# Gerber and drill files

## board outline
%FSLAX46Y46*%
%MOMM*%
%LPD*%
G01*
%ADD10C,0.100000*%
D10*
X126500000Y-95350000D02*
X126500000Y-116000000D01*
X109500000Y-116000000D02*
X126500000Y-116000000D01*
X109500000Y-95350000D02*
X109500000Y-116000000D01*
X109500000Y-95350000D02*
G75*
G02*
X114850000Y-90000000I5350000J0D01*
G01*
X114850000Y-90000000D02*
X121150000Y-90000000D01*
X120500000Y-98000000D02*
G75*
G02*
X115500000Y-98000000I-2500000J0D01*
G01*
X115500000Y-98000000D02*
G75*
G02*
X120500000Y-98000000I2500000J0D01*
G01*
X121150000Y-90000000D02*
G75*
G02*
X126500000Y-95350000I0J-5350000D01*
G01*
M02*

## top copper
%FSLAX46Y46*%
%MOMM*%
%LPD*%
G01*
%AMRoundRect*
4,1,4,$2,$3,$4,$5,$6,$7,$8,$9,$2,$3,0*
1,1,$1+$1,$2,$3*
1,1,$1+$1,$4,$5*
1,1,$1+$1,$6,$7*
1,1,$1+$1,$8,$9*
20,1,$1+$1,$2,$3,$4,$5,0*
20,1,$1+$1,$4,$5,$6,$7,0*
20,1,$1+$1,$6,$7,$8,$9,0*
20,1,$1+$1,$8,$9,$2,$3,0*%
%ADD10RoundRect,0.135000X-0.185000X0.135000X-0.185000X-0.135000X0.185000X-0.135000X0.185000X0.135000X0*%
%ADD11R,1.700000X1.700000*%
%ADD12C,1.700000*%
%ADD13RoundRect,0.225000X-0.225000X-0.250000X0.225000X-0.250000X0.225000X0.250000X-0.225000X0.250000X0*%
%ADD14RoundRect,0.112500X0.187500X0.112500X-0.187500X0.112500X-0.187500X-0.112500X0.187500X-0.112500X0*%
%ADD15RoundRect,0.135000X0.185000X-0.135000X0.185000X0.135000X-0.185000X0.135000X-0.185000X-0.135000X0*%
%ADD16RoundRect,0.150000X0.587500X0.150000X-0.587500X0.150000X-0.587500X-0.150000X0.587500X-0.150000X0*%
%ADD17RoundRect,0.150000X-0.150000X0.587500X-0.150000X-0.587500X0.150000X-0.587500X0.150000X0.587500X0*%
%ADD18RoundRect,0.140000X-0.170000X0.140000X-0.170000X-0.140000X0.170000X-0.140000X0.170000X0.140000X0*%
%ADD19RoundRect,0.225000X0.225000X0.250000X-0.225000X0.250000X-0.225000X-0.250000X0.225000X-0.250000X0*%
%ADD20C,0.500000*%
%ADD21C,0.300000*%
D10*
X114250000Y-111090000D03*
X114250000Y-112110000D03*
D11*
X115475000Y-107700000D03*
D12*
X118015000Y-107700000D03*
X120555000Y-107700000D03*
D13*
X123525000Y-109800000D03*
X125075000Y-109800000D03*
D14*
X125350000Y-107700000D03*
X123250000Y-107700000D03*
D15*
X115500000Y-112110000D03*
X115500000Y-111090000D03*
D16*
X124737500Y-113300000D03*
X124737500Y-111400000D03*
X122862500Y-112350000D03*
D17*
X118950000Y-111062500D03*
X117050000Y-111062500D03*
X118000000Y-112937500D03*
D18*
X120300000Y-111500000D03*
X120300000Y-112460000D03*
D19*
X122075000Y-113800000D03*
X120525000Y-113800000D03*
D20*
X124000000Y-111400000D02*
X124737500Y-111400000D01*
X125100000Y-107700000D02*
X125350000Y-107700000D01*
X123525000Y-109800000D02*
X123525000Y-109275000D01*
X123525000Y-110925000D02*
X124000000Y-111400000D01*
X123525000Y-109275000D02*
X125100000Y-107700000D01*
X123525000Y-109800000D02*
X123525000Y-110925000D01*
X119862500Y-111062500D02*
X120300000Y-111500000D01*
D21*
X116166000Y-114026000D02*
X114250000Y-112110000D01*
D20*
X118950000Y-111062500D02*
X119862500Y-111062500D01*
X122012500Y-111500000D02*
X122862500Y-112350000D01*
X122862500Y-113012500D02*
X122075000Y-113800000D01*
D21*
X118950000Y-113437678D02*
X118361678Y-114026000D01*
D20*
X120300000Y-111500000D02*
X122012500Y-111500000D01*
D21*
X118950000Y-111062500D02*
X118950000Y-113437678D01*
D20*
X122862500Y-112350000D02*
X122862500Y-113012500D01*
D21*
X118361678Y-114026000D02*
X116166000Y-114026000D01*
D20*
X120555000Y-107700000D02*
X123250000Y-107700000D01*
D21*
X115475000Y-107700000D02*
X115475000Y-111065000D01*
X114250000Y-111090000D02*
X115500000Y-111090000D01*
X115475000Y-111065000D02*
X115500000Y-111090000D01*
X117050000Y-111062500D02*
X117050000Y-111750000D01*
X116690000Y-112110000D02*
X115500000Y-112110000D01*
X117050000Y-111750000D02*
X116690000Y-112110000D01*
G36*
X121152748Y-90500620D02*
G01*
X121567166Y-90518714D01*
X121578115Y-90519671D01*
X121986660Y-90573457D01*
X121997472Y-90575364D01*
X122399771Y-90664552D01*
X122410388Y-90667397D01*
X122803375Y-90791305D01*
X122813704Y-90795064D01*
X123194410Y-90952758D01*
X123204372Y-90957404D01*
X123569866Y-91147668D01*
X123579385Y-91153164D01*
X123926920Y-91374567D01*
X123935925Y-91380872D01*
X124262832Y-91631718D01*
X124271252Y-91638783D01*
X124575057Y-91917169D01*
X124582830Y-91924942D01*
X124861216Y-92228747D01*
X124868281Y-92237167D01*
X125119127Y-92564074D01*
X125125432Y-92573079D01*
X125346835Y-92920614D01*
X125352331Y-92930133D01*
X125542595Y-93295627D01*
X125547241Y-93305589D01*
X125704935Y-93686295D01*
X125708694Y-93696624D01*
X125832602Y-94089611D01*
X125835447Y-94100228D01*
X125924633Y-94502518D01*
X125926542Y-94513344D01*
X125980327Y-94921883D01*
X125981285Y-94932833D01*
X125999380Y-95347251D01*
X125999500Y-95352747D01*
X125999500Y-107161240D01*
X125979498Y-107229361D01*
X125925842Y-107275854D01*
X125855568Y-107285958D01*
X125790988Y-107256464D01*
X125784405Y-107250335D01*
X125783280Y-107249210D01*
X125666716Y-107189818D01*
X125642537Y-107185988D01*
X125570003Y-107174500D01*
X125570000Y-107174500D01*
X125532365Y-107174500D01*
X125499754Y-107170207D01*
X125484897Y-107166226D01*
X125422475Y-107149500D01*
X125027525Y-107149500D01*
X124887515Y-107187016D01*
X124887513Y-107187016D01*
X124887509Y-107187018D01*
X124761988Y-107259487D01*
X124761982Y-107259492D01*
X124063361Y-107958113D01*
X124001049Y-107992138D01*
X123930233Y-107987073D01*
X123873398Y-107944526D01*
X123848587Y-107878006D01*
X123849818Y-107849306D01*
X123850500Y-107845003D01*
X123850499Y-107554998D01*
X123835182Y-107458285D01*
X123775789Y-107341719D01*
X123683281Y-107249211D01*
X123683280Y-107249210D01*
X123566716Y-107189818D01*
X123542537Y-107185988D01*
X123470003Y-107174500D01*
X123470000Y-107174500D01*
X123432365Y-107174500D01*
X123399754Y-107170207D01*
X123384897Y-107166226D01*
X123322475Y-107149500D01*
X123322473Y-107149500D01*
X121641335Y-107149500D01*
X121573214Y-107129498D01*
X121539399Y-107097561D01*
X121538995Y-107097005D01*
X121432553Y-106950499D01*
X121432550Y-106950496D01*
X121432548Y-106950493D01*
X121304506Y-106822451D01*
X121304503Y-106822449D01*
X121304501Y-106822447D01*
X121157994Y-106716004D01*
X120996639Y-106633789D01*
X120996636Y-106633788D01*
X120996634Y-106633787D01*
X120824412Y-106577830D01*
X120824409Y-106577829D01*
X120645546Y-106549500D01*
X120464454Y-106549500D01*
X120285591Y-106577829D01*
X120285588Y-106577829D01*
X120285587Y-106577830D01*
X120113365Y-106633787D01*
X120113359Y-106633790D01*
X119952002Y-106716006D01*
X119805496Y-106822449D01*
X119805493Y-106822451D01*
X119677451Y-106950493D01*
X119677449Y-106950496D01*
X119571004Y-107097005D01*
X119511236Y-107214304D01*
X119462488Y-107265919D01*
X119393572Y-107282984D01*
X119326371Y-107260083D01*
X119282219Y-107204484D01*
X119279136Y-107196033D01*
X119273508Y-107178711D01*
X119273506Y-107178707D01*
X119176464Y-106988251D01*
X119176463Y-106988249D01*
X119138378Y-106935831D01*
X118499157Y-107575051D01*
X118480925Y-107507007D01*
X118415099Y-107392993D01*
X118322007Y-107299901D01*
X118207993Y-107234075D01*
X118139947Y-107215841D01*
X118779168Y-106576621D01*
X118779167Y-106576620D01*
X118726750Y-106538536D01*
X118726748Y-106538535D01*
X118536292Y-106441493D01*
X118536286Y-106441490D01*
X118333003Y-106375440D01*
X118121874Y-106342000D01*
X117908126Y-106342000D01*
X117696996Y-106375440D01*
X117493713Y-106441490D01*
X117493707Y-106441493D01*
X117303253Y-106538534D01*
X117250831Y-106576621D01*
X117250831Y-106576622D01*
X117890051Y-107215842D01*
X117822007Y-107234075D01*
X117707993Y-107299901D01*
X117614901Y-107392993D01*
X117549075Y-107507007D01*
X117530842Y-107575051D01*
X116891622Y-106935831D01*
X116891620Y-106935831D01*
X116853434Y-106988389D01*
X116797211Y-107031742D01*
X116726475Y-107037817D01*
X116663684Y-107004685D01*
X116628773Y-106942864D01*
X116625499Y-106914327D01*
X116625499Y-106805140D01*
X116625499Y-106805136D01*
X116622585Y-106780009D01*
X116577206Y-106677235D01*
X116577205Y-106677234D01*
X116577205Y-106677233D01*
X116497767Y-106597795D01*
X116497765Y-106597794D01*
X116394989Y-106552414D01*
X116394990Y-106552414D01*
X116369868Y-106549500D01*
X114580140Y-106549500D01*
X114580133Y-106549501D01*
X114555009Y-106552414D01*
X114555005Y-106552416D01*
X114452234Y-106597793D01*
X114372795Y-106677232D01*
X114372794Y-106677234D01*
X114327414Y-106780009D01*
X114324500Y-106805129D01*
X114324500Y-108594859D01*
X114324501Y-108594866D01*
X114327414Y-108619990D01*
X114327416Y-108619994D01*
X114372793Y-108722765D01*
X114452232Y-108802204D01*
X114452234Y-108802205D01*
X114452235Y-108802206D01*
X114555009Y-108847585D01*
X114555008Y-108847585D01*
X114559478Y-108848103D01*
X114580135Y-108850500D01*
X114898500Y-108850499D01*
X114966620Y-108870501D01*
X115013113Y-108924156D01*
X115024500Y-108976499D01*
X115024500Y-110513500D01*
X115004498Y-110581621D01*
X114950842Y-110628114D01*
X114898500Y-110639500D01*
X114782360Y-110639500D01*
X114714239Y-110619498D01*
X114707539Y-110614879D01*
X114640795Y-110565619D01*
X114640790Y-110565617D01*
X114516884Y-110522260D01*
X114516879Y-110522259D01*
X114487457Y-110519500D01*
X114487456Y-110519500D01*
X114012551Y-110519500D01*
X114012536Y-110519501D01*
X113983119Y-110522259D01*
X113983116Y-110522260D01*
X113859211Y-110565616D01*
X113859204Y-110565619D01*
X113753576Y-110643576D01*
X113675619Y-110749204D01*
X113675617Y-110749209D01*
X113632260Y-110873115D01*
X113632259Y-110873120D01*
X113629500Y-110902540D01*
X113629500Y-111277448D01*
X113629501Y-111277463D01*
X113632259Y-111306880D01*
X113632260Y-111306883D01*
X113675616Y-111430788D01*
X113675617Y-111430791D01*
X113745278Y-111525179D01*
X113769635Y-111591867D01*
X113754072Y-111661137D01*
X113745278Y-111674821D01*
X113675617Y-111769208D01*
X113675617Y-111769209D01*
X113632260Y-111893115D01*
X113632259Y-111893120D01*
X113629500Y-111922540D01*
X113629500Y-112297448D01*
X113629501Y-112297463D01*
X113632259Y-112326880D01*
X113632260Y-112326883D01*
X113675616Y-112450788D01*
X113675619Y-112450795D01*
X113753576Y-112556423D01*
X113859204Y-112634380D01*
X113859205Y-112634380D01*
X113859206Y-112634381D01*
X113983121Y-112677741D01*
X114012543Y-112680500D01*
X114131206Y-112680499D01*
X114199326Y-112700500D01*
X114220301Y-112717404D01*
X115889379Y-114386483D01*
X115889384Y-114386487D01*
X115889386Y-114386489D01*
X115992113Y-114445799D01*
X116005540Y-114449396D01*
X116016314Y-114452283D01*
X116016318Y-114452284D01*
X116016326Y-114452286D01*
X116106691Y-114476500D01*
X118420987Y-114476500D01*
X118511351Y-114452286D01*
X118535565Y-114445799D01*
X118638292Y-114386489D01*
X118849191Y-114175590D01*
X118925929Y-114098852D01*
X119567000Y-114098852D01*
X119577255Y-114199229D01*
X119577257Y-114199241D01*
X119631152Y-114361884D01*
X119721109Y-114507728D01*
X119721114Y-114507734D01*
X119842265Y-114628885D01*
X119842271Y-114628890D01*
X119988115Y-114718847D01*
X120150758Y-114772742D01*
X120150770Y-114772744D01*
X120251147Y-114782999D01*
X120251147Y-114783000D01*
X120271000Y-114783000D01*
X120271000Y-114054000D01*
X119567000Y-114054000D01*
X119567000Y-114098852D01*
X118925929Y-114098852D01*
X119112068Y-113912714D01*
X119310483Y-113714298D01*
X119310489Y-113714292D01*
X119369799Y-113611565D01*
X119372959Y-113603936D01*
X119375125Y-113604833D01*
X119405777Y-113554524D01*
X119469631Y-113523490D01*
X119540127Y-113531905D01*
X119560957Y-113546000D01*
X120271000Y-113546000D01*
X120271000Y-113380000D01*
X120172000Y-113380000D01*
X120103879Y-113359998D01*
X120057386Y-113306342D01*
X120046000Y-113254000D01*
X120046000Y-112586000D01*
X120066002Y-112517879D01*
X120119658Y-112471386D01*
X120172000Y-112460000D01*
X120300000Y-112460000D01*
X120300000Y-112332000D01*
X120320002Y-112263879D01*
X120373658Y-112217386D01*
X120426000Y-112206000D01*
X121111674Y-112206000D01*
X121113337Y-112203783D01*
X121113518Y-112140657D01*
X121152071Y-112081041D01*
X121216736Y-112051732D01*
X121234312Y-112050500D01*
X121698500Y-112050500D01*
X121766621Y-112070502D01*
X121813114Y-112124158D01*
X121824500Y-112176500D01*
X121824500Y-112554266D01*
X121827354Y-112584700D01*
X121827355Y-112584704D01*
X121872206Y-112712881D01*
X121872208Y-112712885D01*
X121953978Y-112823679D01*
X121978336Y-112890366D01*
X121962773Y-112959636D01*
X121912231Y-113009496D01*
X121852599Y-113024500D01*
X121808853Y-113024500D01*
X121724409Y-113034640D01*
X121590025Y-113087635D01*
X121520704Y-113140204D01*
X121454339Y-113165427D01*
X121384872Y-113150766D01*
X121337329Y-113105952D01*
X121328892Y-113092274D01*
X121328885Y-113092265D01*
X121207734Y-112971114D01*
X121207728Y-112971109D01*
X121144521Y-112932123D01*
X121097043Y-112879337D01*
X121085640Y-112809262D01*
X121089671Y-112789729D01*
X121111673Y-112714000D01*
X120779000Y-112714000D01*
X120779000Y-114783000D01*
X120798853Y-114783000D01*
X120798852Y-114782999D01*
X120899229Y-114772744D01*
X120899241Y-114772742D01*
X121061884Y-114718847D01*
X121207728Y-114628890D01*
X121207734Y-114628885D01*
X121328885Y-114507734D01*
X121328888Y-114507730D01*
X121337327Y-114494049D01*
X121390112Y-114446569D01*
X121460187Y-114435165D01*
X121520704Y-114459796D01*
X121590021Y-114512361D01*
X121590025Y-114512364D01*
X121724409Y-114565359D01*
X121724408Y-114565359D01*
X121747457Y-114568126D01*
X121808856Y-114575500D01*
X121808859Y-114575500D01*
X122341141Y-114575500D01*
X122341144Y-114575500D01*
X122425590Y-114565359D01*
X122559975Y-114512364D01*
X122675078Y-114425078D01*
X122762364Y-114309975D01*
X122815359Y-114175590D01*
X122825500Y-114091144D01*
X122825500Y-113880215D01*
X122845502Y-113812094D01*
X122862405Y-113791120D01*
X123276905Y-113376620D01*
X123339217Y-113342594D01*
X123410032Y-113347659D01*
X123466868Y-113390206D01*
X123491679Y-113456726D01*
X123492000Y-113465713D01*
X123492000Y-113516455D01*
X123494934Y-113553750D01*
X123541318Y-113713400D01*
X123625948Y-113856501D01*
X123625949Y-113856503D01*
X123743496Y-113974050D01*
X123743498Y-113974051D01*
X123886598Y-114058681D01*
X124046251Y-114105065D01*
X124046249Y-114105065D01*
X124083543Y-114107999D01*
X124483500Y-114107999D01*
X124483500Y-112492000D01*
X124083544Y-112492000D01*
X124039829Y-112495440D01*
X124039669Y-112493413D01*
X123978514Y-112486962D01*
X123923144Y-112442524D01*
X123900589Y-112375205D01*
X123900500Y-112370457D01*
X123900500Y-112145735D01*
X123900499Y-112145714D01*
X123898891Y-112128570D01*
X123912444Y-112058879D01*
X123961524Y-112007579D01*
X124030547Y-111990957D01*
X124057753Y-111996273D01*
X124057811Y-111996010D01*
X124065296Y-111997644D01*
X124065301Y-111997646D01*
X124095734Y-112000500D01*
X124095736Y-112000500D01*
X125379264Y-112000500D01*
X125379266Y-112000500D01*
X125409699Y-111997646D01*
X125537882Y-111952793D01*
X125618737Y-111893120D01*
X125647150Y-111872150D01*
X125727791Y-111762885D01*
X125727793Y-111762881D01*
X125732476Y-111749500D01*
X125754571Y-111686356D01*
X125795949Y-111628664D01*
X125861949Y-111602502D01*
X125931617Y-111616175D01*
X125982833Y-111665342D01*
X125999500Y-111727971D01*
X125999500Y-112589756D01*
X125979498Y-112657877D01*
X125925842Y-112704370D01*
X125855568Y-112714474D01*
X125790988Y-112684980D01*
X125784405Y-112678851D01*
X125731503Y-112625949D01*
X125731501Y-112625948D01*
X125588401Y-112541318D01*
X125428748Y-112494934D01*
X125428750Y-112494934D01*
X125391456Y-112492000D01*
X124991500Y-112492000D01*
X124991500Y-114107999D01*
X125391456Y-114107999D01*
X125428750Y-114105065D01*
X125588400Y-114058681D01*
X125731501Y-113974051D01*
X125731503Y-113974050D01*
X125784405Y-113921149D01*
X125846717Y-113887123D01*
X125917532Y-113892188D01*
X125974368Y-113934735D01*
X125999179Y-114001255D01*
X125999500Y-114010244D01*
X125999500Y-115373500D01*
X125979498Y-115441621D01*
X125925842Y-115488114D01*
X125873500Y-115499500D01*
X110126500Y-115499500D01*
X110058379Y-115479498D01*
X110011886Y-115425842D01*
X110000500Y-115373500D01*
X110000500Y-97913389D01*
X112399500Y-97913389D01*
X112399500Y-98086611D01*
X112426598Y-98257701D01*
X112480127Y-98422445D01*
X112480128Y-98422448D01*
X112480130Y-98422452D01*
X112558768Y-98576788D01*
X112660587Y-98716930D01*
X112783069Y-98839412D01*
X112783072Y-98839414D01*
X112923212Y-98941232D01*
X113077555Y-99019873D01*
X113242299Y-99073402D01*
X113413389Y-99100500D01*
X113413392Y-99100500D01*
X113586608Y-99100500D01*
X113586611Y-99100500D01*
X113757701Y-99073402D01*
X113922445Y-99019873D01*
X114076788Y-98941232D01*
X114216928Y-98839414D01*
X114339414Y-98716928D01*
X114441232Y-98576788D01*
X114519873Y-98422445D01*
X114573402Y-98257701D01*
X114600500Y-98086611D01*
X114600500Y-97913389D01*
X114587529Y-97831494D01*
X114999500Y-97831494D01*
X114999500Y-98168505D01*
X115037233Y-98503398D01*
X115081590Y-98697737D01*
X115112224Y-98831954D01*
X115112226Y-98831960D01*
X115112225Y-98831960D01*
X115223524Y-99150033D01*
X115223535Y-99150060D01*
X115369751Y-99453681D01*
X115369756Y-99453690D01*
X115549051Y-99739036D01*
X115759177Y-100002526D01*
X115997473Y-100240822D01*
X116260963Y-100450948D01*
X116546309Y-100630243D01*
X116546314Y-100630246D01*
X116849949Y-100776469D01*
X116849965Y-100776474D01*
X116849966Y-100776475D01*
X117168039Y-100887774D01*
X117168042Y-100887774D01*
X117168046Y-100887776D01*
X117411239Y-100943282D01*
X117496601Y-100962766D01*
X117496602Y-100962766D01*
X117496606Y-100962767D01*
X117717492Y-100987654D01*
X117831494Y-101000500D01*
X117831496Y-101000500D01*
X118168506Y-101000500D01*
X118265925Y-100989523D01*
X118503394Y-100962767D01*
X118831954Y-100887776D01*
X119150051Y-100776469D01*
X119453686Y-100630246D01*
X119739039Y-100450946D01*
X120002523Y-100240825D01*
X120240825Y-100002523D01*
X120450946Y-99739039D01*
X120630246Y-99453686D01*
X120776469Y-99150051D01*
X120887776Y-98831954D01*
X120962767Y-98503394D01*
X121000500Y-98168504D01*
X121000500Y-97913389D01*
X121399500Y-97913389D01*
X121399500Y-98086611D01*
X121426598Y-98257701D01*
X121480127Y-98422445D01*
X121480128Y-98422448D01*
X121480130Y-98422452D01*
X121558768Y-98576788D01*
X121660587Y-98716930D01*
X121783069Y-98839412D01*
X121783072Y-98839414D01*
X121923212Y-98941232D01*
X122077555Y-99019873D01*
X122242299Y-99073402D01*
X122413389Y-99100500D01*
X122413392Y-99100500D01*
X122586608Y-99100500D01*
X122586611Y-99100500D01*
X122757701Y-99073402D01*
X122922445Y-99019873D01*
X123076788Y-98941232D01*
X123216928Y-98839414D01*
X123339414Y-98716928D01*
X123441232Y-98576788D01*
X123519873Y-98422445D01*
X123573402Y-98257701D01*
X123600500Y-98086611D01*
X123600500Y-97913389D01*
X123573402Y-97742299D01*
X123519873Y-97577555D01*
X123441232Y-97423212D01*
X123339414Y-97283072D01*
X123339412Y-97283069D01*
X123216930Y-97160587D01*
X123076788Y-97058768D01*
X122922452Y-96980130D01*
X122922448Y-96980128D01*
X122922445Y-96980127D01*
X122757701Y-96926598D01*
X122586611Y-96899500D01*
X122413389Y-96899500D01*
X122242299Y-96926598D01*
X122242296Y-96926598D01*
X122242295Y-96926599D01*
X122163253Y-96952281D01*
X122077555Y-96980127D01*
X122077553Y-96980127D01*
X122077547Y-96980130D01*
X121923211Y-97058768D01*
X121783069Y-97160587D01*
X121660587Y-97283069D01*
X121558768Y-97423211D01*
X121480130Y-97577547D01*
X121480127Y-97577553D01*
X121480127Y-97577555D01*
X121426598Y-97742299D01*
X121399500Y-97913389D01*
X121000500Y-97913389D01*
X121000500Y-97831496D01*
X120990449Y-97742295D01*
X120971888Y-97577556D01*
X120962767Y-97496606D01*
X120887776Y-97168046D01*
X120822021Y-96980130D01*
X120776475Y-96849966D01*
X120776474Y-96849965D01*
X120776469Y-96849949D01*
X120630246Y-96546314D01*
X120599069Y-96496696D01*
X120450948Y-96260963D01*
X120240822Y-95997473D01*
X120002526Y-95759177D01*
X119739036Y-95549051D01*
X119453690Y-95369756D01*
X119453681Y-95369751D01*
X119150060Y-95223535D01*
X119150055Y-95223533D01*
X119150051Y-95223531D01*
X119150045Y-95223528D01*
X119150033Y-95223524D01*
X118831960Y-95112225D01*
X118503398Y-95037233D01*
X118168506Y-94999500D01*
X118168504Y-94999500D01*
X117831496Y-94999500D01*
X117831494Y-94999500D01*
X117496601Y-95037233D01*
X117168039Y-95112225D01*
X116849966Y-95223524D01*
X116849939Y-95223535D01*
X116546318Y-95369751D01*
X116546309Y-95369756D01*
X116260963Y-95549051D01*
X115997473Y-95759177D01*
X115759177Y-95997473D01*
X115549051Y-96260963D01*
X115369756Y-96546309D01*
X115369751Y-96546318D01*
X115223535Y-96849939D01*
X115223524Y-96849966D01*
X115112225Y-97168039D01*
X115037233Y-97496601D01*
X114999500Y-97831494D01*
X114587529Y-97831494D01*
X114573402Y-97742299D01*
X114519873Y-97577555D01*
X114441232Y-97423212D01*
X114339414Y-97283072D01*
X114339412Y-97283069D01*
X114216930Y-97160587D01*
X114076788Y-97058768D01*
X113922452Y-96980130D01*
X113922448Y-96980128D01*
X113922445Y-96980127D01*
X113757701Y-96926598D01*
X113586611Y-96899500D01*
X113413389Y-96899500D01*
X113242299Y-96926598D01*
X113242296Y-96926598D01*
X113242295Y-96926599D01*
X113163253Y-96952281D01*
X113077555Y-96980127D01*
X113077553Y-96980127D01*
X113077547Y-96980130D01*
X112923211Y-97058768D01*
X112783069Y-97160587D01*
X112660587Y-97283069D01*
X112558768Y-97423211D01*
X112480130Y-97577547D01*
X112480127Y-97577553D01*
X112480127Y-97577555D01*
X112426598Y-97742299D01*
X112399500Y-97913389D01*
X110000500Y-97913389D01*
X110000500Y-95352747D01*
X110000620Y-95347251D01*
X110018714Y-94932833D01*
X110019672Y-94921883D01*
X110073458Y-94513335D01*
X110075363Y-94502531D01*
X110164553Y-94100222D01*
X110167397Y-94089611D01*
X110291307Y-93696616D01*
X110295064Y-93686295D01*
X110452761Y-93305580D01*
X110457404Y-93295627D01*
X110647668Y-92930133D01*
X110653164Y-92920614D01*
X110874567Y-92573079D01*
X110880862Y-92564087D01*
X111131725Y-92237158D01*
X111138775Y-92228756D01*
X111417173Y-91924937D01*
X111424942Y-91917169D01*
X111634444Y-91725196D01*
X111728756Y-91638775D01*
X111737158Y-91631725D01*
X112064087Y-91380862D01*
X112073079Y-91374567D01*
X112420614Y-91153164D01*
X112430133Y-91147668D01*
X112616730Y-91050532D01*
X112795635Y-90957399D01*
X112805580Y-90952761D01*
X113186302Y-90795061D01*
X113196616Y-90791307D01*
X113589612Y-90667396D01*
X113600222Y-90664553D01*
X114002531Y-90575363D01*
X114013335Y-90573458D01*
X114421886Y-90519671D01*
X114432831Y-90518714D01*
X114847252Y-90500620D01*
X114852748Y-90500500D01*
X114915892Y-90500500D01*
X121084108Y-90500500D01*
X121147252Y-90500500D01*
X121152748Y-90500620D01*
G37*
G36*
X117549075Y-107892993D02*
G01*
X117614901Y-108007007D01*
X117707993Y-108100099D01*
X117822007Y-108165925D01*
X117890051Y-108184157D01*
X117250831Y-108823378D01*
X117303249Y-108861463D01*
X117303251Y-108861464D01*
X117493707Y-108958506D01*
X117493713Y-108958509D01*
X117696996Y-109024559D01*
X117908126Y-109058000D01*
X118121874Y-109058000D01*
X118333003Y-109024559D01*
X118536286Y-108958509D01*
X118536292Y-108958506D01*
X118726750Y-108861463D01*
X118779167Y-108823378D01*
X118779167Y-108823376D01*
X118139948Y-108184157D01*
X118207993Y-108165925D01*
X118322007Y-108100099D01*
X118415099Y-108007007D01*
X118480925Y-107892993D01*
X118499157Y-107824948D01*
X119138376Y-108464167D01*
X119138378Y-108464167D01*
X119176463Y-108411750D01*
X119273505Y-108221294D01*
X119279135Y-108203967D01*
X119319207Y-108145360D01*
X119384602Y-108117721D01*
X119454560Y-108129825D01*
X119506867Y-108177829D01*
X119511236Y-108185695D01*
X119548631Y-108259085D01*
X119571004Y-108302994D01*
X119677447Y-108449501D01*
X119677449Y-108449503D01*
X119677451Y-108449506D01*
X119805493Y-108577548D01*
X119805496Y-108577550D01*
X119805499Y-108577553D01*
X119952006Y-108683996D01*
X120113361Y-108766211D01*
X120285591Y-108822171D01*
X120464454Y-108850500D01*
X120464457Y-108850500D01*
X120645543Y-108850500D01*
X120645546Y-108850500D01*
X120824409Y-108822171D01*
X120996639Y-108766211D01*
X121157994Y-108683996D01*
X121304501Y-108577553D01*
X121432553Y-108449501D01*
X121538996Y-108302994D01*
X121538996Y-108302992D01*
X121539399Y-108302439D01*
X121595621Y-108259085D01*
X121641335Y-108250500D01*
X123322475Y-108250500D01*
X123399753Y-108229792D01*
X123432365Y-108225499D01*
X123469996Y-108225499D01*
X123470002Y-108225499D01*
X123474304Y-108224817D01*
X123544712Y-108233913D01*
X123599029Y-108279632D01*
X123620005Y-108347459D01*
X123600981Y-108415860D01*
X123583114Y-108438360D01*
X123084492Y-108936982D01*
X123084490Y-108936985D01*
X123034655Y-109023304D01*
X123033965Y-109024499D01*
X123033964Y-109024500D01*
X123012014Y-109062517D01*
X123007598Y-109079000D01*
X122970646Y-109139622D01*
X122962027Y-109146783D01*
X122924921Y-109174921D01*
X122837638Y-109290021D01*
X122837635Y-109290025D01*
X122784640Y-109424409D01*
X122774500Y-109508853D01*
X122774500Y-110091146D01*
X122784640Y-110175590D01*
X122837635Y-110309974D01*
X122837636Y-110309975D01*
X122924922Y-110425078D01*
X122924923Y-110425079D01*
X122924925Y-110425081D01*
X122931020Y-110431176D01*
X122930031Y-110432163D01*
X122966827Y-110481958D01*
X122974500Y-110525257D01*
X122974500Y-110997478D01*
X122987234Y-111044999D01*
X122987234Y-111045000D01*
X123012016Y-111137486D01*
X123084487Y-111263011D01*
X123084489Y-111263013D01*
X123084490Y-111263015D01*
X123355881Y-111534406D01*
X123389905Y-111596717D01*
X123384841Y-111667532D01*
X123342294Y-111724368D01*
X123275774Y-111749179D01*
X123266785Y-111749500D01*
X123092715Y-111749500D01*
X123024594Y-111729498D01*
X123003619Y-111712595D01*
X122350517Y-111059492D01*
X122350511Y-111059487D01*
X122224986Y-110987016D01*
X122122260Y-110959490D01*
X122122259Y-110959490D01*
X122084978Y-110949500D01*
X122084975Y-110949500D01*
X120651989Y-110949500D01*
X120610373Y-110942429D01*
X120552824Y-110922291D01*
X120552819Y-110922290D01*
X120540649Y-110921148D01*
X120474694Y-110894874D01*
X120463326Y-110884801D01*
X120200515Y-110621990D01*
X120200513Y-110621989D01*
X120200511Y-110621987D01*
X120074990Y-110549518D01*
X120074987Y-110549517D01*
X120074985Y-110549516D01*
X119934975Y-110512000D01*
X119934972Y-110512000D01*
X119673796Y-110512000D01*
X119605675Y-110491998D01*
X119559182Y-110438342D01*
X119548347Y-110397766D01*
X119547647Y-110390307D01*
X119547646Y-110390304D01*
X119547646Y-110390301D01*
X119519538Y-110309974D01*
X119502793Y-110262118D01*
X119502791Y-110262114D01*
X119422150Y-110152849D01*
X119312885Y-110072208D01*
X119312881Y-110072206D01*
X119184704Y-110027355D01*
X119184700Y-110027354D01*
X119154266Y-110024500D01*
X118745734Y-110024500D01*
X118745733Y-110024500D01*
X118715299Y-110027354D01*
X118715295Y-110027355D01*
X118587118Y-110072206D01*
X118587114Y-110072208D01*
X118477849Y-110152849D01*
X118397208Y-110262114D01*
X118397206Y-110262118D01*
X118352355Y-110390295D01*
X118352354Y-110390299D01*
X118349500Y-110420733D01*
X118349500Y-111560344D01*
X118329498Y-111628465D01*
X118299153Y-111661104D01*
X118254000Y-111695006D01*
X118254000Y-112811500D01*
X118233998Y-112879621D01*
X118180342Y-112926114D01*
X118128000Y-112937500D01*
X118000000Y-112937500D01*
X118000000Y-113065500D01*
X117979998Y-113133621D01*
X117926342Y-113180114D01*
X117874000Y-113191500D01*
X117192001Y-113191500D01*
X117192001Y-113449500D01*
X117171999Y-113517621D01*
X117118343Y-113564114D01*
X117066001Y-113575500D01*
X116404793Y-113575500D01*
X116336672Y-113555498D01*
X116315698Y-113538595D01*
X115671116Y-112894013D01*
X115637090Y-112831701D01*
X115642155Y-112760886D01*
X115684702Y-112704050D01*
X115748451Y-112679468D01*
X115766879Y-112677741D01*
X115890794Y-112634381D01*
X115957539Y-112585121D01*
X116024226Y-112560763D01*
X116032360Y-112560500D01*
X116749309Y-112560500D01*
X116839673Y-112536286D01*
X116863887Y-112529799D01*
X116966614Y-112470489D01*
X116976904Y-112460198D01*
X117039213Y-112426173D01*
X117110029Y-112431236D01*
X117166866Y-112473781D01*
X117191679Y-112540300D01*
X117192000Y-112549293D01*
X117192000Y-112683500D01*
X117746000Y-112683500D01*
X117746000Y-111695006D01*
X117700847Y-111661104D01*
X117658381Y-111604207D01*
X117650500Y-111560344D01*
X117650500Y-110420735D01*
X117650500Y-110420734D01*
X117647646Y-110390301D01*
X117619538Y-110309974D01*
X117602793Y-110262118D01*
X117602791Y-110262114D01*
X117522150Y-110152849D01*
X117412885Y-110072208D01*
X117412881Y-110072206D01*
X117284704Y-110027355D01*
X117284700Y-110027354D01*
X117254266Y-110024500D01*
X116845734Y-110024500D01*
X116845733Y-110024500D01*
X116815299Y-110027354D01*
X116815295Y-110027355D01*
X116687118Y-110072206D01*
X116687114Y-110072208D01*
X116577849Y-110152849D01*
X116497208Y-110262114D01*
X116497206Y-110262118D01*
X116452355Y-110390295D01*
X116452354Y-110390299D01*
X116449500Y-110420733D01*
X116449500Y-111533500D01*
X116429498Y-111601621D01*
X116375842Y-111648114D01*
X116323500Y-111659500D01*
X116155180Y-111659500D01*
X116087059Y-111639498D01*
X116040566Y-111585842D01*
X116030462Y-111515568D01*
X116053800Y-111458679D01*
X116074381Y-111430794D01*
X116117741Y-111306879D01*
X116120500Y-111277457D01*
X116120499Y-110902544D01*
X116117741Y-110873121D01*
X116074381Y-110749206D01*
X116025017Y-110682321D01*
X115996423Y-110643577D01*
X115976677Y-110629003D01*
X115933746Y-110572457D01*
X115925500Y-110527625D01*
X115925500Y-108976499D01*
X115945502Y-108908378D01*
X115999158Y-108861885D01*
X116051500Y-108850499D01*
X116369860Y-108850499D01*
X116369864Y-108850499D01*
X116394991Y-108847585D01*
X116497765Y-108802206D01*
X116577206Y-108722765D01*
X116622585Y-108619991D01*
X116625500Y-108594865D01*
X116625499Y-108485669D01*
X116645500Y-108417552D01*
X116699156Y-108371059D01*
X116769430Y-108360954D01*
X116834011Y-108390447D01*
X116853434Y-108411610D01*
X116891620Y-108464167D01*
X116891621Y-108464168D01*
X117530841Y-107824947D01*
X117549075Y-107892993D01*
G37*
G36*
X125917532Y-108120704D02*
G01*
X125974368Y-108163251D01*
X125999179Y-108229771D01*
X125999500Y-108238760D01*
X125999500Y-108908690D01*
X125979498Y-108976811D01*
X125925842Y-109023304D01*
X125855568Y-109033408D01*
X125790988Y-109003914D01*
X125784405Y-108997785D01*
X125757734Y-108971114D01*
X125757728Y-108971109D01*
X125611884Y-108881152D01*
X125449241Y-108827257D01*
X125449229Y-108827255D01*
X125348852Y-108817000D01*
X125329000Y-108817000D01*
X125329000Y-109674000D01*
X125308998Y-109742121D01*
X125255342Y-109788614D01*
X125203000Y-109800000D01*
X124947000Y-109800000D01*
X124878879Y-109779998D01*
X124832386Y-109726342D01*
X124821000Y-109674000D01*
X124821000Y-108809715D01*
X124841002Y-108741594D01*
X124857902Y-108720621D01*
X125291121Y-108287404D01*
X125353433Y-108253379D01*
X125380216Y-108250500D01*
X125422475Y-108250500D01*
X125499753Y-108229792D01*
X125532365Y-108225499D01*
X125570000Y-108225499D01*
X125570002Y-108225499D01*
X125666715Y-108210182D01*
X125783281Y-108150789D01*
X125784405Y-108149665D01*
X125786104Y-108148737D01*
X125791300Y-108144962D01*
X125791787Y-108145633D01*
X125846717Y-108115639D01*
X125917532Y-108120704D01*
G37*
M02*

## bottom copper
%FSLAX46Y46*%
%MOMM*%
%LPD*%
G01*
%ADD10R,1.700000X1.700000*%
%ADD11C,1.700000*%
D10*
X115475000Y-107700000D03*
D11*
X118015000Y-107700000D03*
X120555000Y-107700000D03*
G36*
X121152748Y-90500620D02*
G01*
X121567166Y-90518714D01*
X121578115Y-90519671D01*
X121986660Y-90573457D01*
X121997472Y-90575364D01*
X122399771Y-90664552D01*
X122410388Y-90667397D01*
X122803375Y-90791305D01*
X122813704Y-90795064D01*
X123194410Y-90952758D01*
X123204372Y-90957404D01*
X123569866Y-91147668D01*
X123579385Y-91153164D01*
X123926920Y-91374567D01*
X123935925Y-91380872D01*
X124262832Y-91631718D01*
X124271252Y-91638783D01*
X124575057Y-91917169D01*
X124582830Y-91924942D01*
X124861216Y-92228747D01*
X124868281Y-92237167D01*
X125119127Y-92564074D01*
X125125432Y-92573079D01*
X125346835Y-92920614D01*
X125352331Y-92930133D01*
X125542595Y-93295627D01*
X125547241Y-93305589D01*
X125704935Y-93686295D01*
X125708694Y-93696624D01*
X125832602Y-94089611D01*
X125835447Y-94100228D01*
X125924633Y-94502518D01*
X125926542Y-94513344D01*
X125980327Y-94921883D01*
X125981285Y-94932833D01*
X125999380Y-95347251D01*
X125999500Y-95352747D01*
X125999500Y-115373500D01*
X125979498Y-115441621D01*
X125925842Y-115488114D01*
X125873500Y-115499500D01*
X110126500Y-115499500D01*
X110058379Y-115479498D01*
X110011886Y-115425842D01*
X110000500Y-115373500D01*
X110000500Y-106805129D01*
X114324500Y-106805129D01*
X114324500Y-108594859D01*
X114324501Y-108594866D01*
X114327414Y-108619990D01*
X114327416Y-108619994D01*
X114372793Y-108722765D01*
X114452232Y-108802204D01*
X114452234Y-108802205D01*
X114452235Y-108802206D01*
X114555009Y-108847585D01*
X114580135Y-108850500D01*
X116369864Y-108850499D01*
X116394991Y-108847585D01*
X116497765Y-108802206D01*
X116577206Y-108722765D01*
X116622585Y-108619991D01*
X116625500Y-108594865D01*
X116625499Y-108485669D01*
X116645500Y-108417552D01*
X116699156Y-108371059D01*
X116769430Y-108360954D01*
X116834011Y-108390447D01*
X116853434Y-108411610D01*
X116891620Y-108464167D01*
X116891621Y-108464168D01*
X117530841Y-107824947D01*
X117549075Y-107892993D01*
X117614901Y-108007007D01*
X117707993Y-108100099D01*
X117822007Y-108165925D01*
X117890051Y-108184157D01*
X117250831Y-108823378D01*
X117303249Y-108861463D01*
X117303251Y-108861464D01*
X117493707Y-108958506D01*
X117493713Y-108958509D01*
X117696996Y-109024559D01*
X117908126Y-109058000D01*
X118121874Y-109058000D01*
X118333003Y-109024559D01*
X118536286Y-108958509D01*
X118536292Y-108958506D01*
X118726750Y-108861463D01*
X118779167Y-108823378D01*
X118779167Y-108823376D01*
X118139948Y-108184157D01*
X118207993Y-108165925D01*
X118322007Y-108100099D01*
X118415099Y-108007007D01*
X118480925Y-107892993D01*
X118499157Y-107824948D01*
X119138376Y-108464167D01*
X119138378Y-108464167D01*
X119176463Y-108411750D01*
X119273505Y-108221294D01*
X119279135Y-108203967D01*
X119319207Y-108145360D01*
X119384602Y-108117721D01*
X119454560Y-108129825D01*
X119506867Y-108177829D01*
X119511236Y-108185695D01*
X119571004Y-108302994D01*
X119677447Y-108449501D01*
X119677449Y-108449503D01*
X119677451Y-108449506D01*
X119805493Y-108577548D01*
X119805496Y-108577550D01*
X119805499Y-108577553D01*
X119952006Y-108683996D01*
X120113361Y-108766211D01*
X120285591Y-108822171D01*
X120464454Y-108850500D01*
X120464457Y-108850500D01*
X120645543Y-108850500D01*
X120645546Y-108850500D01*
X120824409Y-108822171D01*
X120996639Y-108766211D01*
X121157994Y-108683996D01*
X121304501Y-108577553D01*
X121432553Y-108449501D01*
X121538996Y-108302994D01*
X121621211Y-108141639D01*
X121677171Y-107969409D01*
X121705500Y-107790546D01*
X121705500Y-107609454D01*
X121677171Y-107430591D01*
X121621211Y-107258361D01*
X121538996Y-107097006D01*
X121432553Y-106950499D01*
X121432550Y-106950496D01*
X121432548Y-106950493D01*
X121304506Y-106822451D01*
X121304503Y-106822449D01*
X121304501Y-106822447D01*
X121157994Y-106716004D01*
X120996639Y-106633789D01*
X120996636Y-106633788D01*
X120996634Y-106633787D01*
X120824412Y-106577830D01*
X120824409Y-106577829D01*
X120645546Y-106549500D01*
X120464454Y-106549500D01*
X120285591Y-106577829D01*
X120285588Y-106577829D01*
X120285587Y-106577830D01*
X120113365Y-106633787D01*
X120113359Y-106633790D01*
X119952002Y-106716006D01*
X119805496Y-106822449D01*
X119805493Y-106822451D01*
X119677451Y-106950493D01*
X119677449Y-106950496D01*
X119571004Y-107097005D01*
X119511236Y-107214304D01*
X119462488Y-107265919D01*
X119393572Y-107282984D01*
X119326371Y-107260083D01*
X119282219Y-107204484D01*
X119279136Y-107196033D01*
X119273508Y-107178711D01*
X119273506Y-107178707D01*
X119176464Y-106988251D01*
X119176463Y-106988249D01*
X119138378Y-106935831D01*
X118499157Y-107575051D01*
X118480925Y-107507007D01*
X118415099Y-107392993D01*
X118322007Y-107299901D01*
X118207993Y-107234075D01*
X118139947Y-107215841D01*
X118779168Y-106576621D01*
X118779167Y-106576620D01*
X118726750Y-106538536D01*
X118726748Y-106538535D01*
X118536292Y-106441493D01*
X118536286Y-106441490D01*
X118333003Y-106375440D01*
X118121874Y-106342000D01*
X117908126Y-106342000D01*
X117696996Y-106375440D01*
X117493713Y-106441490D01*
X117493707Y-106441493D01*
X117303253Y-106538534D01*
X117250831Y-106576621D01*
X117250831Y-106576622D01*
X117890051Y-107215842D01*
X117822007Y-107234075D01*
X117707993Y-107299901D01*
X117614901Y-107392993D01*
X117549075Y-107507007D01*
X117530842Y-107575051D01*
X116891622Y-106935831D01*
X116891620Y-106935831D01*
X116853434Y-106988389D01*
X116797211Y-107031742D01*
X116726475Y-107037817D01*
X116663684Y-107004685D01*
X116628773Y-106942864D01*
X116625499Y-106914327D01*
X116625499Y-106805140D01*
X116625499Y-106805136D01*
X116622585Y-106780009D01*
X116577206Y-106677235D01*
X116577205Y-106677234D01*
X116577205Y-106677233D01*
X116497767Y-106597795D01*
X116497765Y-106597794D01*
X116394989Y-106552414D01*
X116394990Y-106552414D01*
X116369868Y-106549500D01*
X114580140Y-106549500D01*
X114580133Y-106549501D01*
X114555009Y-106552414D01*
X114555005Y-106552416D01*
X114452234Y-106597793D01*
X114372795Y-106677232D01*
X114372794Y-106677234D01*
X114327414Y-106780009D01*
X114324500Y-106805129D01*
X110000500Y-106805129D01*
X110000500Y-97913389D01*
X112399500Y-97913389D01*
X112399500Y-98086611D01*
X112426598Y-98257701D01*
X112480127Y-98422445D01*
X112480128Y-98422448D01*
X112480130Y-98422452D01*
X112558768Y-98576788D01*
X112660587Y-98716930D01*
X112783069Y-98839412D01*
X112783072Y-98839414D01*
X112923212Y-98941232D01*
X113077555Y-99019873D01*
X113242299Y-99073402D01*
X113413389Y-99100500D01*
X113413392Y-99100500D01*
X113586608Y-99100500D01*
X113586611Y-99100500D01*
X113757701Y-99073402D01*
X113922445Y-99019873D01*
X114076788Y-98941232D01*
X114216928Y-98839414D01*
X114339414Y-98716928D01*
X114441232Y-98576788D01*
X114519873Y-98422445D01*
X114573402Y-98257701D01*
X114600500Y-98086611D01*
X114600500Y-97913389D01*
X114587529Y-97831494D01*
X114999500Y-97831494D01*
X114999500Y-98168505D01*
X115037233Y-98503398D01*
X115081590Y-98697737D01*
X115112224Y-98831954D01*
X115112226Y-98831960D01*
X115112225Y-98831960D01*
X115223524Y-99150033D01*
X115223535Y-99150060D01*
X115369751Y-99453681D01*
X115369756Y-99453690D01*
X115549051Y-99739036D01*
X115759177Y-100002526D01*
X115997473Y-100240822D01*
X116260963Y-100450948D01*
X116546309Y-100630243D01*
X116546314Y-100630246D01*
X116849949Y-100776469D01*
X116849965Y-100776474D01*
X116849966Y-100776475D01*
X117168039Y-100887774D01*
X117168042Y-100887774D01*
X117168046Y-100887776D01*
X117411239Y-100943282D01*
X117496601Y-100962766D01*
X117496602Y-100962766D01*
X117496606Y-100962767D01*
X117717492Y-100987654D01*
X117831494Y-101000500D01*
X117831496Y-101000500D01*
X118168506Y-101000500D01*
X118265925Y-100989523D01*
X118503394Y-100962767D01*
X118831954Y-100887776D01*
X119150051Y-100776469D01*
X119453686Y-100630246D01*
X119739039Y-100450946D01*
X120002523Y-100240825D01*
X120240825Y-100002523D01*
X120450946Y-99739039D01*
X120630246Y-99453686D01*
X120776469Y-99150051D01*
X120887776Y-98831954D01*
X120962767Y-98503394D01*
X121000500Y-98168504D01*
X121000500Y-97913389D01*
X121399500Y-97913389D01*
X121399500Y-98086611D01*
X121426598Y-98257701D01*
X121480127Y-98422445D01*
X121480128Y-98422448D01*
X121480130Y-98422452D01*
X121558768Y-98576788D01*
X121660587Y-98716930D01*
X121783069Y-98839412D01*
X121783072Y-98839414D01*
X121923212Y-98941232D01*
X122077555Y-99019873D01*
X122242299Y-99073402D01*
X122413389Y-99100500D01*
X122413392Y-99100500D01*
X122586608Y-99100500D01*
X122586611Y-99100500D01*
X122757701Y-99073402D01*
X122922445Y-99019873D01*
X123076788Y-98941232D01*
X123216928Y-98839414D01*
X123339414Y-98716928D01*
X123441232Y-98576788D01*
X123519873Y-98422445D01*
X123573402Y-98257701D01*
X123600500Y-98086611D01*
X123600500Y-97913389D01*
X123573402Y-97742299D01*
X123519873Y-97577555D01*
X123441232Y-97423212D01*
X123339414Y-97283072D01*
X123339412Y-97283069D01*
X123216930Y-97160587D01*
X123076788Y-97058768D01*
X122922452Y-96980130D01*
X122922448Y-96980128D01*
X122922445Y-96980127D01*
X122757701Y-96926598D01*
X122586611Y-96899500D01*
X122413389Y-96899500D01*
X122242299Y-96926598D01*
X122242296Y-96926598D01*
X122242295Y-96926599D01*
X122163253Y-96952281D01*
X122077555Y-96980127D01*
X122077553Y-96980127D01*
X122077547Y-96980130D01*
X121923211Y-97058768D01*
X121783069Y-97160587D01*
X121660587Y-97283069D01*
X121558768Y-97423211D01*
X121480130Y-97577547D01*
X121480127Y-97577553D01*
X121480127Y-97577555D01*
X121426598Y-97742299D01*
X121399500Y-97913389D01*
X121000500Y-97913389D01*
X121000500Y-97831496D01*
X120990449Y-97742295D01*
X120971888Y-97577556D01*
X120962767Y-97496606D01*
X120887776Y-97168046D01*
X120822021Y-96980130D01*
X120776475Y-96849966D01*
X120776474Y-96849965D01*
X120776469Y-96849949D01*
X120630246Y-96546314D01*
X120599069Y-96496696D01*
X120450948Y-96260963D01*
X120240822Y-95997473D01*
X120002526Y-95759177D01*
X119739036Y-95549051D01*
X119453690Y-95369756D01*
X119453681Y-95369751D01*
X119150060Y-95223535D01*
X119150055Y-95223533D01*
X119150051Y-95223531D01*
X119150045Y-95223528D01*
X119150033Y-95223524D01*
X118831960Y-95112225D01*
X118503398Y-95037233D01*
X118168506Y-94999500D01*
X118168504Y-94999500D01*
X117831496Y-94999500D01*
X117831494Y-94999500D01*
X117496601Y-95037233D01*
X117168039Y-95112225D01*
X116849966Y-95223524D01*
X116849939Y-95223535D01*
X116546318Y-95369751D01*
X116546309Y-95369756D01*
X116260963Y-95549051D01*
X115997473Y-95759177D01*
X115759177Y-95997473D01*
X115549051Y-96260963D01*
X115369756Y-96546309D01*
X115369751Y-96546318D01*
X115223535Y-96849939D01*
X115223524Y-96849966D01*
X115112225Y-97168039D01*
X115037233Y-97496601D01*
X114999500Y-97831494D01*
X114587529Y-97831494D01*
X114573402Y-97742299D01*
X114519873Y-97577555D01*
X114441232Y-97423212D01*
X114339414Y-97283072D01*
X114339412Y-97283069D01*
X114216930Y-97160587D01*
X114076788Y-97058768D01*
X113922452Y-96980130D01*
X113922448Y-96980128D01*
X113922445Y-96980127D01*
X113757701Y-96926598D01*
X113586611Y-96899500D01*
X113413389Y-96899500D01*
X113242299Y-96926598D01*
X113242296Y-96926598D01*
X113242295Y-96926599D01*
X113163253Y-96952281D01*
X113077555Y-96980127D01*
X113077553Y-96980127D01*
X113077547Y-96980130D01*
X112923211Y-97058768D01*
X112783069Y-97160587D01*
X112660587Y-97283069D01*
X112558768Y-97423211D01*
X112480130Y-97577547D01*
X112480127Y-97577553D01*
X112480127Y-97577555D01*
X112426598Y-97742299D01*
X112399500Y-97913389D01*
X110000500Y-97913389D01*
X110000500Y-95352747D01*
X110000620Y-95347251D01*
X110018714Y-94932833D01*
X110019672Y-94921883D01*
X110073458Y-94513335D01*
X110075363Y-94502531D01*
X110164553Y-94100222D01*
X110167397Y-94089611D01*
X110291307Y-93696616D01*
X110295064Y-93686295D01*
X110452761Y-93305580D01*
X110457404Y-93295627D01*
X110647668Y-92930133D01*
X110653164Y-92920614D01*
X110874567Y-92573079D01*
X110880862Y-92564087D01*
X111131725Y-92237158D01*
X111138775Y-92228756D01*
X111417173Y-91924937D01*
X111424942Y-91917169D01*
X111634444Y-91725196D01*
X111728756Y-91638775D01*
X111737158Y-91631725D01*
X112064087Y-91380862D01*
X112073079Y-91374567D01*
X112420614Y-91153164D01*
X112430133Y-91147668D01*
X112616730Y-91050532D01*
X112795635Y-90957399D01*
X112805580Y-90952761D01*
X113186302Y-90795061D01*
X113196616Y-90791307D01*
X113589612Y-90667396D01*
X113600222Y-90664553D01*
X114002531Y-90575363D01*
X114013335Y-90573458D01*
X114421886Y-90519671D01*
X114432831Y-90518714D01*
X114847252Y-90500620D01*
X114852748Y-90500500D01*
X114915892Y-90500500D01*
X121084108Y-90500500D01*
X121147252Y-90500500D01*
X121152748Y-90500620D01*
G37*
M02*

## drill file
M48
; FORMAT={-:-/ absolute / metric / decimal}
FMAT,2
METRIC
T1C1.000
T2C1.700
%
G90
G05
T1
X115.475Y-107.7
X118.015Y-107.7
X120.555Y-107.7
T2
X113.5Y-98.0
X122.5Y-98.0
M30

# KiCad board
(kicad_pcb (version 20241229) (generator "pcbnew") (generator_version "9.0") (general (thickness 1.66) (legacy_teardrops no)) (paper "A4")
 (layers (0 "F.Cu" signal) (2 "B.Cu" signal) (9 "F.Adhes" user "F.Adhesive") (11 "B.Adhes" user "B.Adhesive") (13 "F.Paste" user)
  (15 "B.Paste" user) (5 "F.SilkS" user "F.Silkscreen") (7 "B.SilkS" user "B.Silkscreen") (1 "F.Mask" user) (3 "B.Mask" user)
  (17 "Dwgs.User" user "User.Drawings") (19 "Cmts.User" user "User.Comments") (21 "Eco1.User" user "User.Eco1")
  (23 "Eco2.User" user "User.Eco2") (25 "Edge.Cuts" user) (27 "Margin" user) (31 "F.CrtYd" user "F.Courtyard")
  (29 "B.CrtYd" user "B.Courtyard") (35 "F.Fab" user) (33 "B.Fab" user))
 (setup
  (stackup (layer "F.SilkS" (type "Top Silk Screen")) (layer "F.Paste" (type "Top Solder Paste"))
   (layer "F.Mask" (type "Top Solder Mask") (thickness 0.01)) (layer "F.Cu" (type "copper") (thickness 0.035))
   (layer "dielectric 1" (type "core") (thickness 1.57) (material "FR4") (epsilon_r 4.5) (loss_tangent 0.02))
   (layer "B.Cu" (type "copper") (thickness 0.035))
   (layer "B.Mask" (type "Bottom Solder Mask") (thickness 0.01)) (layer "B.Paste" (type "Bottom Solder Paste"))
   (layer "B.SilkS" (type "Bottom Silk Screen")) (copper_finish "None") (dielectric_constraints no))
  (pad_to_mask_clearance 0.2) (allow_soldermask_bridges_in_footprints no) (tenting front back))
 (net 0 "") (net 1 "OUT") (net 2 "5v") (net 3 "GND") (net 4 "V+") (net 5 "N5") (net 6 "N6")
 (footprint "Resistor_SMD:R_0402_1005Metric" (layer "F.Cu") (at 114.25 111.6 -90)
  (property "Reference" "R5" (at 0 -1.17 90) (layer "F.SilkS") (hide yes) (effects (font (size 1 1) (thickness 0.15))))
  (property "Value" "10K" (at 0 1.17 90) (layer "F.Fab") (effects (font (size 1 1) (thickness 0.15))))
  (pad "1" smd roundrect (at -0.51 0 270) (size 0.54 0.64) (layers "F.Cu" "F.Mask" "F.Paste") (roundrect_rratio 0.25) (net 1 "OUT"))
  (pad "2" smd roundrect (at 0.51 0 270) (size 0.54 0.64) (layers "F.Cu" "F.Mask" "F.Paste") (roundrect_rratio 0.25) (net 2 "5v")))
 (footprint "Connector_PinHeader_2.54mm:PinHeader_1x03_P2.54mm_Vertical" (layer "F.Cu") (at 115.475 107.7 90)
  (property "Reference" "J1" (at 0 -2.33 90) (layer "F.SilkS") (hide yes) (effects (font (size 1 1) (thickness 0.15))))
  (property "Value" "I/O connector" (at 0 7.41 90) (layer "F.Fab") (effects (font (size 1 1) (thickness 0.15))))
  (pad "1" thru_hole rect (at 0 0 90) (size 1.7 1.7) (drill 1) (layers "*.Cu" "*.Mask") (remove_unused_layers no) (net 1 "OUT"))
  (pad "2" thru_hole circle (at 0 2.54 90) (size 1.7 1.7) (drill 1) (layers "*.Cu" "*.Mask") (remove_unused_layers no) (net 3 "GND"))
  (pad "3" thru_hole circle (at 0 5.08 90) (size 1.7 1.7) (drill 1) (layers "*.Cu" "*.Mask") (remove_unused_layers no) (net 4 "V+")))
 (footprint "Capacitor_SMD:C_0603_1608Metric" (layer "F.Cu") (at 124.3 109.8)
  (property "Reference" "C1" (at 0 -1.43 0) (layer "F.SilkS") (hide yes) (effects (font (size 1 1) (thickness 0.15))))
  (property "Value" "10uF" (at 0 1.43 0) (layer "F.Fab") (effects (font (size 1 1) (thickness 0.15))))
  (pad "1" smd roundrect (at -0.775 0) (size 0.9 0.95) (layers "F.Cu" "F.Mask" "F.Paste") (roundrect_rratio 0.25) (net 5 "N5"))
  (pad "2" smd roundrect (at 0.775 0) (size 0.9 0.95) (layers "F.Cu" "F.Mask" "F.Paste") (roundrect_rratio 0.25) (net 3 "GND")))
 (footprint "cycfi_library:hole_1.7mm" (layer "F.Cu") (at 122.5 98)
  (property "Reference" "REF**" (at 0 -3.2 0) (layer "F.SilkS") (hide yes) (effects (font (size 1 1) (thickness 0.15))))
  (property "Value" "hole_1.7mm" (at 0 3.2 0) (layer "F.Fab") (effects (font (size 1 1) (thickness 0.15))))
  (pad "" np_thru_hole circle (at 0 0) (size 1.7 1.7) (drill 1.7) (layers "*.Cu" "*.Mask")))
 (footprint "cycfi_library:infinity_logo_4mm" (layer "F.Cu") (at 111.3 108.4 -90)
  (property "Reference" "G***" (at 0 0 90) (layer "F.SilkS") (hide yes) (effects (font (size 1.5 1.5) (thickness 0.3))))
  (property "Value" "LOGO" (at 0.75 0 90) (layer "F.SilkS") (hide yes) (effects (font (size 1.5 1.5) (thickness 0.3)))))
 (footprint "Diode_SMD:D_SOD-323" (layer "F.Cu") (at 124.3 107.7 180)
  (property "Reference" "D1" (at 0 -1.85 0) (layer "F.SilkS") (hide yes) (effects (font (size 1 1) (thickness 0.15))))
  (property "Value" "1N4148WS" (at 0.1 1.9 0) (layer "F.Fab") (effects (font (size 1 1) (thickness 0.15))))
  (pad "1" smd roundrect (at -1.05 0 180) (size 0.6 0.45) (layers "F.Cu" "F.Mask" "F.Paste") (roundrect_rratio 0.25) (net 5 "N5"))
  (pad "2" smd roundrect (at 1.05 0 180) (size 0.6 0.45) (layers "F.Cu" "F.Mask" "F.Paste") (roundrect_rratio 0.25) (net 4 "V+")))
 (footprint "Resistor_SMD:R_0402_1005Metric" (layer "F.Cu") (at 115.5 111.6 90)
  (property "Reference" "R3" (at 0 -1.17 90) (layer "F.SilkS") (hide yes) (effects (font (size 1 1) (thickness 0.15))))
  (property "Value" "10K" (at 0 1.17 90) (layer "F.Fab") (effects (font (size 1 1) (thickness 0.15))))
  (pad "1" smd roundrect (at -0.51 0 90) (size 0.54 0.64) (layers "F.Cu" "F.Mask" "F.Paste") (roundrect_rratio 0.25) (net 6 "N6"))
  (pad "2" smd roundrect (at 0.51 0 90) (size 0.54 0.64) (layers "F.Cu" "F.Mask" "F.Paste") (roundrect_rratio 0.25) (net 1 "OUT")))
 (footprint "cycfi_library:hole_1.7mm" (layer "F.Cu") (at 113.5 98)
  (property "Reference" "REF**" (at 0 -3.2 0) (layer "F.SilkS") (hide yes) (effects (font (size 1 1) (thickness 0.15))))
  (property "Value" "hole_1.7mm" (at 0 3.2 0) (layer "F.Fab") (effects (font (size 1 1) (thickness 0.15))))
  (pad "" np_thru_hole circle (at 0 0) (size 1.7 1.7) (drill 1.7) (layers "*.Cu" "*.Mask")))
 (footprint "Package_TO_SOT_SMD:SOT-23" (layer "F.Cu") (at 123.8 112.35 180)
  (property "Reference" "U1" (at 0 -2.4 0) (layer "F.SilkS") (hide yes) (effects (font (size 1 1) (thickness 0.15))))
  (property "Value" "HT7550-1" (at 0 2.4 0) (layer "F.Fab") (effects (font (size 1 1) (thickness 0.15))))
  (pad "1" smd roundrect (at -0.9375 -0.95 180) (size 1.475 0.6) (layers "F.Cu" "F.Mask" "F.Paste") (roundrect_rratio 0.25) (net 3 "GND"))
  (pad "2" smd roundrect (at -0.9375 0.95 180) (size 1.475 0.6) (layers "F.Cu" "F.Mask" "F.Paste") (roundrect_rratio 0.25) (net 5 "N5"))
  (pad "3" smd roundrect (at 0.9375 0 180) (size 1.475 0.6) (layers "F.Cu" "F.Mask" "F.Paste") (roundrect_rratio 0.25) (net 2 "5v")))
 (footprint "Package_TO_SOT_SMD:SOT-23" (layer "F.Cu") (at 118 112 -90)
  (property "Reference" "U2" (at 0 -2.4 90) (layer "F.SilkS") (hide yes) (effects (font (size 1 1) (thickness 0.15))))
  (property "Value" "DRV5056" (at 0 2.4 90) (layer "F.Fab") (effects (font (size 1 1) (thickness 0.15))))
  (pad "1" smd roundrect (at -0.9375 -0.95 270) (size 1.475 0.6) (layers "F.Cu" "F.Mask" "F.Paste") (roundrect_rratio 0.25) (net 2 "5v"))
  (pad "2" smd roundrect (at -0.9375 0.95 270) (size 1.475 0.6) (layers "F.Cu" "F.Mask" "F.Paste") (roundrect_rratio 0.25) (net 6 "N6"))
  (pad "3" smd roundrect (at 0.9375 0 270) (size 1.475 0.6) (layers "F.Cu" "F.Mask" "F.Paste") (roundrect_rratio 0.25) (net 3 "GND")))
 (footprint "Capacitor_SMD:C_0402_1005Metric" (layer "F.Cu") (at 120.3 111.98 -90)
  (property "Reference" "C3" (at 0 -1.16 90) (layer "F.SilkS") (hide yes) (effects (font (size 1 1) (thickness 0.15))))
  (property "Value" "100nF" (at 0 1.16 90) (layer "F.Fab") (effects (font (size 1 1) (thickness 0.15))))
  (pad "1" smd roundrect (at -0.48 0 270) (size 0.56 0.62) (layers "F.Cu" "F.Mask" "F.Paste") (roundrect_rratio 0.25) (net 2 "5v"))
  (pad "2" smd roundrect (at 0.48 0 270) (size 0.56 0.62) (layers "F.Cu" "F.Mask" "F.Paste") (roundrect_rratio 0.25) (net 3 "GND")))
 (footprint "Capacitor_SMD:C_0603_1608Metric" (layer "F.Cu") (at 121.3 113.8 180)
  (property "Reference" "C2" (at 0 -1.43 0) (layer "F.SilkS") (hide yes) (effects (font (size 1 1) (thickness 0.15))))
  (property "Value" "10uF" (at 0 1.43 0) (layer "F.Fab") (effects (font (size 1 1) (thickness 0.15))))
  (pad "1" smd roundrect (at -0.775 0 180) (size 0.9 0.95) (layers "F.Cu" "F.Mask" "F.Paste") (roundrect_rratio 0.25) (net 2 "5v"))
  (pad "2" smd roundrect (at 0.775 0 180) (size 0.9 0.95) (layers "F.Cu" "F.Mask" "F.Paste") (roundrect_rratio 0.25) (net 3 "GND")))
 (gr_line (start 126.5 95.35) (end 126.5 116) (stroke (width 0.1) (type default)) (layer "Edge.Cuts"))
 (gr_line (start 109.5 116) (end 126.5 116) (stroke (width 0.1) (type default)) (layer "Edge.Cuts"))
 (gr_line (start 109.5 95.35) (end 109.5 116) (stroke (width 0.1) (type default)) (layer "Edge.Cuts"))
 (gr_arc (start 109.5 95.35) (mid 111.066979 91.566979) (end 114.85 90) (stroke (width 0.1) (type default)) (layer "Edge.Cuts"))
 (gr_line (start 114.85 90) (end 121.15 90) (stroke (width 0.1) (type default)) (layer "Edge.Cuts"))
 (gr_circle (center 118 98) (end 120.5 98) (stroke (width 0.1) (type solid)) (fill no) (layer "Edge.Cuts"))
 (gr_arc (start 121.15 90) (mid 124.933021 91.566979) (end 126.5 95.35) (stroke (width 0.1) (type default)) (layer "Edge.Cuts"))
 (segment (start 124 111.4) (end 124.7375 111.4) (width 0.5) (layer "F.Cu") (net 5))
 (segment (start 125.1 107.7) (end 125.35 107.7) (width 0.5) (layer "F.Cu") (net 5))
 (segment (start 123.525 109.8) (end 123.525 109.275) (width 0.5) (layer "F.Cu") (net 5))
 (segment (start 123.525 110.925) (end 124 111.4) (width 0.5) (layer "F.Cu") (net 5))
 (segment (start 123.525 109.275) (end 125.1 107.7) (width 0.5) (layer "F.Cu") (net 5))
 (segment (start 123.525 109.8) (end 123.525 110.925) (width 0.5) (layer "F.Cu") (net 5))
 (segment (start 119.8625 111.0625) (end 120.3 111.5) (width 0.5) (layer "F.Cu") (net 2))
 (segment (start 116.166 114.026) (end 114.25 112.11) (width 0.3) (layer "F.Cu") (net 2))
 (segment (start 118.95 111.0625) (end 119.8625 111.0625) (width 0.5) (layer "F.Cu") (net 2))
 (segment (start 122.0125 111.5) (end 122.8625 112.35) (width 0.5) (layer "F.Cu") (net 2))
 (segment (start 122.8625 113.0125) (end 122.075 113.8) (width 0.5) (layer "F.Cu") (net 2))
 (segment (start 118.95 113.437678) (end 118.361678 114.026) (width 0.3) (layer "F.Cu") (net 2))
 (segment (start 120.3 111.5) (end 122.0125 111.5) (width 0.5) (layer "F.Cu") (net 2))
 (segment (start 118.95 111.0625) (end 118.95 113.437678) (width 0.3) (layer "F.Cu") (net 2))
 (segment (start 122.8625 112.35) (end 122.8625 113.0125) (width 0.5) (layer "F.Cu") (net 2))
 (segment (start 118.361678 114.026) (end 116.166 114.026) (width 0.3) (layer "F.Cu") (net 2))
 (segment (start 120.555 107.7) (end 123.25 107.7) (width 0.5) (layer "F.Cu") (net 4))
 (segment (start 115.475 107.7) (end 115.475 111.065) (width 0.3) (layer "F.Cu") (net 1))
 (segment (start 114.25 111.09) (end 115.5 111.09) (width 0.3) (layer "F.Cu") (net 1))
 (segment (start 115.475 111.065) (end 115.5 111.09) (width 0.3) (layer "F.Cu") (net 1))
 (segment (start 117.05 111.0625) (end 117.05 111.75) (width 0.3) (layer "F.Cu") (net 6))
 (segment (start 116.69 112.11) (end 115.5 112.11) (width 0.3) (layer "F.Cu") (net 6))
 (segment (start 117.05 111.75) (end 116.69 112.11) (width 0.3) (layer "F.Cu") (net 6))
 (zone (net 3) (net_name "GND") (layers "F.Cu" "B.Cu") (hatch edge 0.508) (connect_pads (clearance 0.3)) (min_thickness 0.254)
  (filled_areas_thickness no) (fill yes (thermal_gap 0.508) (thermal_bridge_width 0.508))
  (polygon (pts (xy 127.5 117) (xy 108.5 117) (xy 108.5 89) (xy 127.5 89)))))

